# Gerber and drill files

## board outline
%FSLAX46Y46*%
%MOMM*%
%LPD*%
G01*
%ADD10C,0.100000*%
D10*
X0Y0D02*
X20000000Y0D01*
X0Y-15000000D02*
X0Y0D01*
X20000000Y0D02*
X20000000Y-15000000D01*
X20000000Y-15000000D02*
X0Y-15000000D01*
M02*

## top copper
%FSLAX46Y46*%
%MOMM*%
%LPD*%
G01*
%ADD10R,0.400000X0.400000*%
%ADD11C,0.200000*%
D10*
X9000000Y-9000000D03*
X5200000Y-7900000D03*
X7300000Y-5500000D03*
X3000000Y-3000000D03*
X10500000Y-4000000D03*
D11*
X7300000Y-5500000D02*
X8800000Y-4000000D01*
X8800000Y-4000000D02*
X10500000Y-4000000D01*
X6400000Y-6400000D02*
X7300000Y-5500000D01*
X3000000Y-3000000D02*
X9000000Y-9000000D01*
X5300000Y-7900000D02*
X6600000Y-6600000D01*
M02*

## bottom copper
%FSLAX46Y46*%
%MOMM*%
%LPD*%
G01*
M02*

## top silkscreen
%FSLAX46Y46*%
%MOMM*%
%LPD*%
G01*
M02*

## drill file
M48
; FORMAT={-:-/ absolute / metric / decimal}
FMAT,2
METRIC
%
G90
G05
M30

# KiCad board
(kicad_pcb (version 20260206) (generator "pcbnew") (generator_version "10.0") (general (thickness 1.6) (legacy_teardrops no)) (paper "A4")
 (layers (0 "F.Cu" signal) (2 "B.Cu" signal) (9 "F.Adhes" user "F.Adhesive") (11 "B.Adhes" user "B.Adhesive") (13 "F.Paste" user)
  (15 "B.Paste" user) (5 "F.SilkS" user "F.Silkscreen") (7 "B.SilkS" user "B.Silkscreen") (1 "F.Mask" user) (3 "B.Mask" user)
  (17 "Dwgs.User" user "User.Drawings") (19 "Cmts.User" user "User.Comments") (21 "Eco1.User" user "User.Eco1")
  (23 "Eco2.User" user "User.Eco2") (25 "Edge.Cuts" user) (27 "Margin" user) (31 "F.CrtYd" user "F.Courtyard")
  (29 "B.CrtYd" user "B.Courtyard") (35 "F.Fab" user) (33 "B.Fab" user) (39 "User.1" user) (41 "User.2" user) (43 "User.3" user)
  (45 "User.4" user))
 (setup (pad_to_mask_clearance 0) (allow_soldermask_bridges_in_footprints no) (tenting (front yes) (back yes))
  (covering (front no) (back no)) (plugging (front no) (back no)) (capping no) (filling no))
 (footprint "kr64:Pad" (layer "F.Cu") (at 9 9)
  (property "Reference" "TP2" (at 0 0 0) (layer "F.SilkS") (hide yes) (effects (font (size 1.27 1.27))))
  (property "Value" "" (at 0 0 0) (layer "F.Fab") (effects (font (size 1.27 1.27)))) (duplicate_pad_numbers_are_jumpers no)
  (pad "1" smd rect (at 0 0) (size 0.4 0.4) (layers "F.Cu" "F.Mask" "F.Paste") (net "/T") (thermal_bridge_angle 45)))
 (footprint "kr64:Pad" (layer "F.Cu") (at 5.2 7.9)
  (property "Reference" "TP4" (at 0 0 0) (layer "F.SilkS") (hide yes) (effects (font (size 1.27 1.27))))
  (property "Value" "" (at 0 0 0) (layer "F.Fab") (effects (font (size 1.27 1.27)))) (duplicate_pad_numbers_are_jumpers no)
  (pad "1" smd rect (at 0 0) (size 0.4 0.4) (layers "F.Cu" "F.Mask" "F.Paste") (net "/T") (thermal_bridge_angle 45)))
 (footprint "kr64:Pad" (layer "F.Cu") (at 7.3 5.5)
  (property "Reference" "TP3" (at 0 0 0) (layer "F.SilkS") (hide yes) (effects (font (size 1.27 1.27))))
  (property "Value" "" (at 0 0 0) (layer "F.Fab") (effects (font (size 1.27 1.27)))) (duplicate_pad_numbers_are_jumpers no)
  (pad "1" smd rect (at 0 0) (size 0.4 0.4) (layers "F.Cu" "F.Mask" "F.Paste") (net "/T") (thermal_bridge_angle 45)))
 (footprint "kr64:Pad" (layer "F.Cu") (at 3 3)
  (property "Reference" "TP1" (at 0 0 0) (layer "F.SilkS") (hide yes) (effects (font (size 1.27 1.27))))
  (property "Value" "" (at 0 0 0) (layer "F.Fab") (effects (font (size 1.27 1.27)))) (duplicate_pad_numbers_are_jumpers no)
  (pad "1" smd rect (at 0 0) (size 0.4 0.4) (layers "F.Cu" "F.Mask" "F.Paste") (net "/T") (thermal_bridge_angle 45)))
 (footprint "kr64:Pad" (layer "F.Cu") (at 10.5 4)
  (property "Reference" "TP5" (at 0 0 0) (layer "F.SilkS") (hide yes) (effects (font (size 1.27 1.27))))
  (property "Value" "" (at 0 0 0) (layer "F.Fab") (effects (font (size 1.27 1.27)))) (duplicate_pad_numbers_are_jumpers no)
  (pad "1" smd rect (at 0 0) (size 0.4 0.4) (layers "F.Cu" "F.Mask" "F.Paste") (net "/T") (thermal_bridge_angle 45)))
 (gr_line (start 0 0) (end 20 0) (stroke (width 0.1) (type default)) (layer "Edge.Cuts"))
 (gr_line (start 0 15) (end 0 0) (stroke (width 0.1) (type default)) (layer "Edge.Cuts"))
 (gr_line (start 20 0) (end 20 15) (stroke (width 0.1) (type default)) (layer "Edge.Cuts"))
 (gr_line (start 20 15) (end 0 15) (stroke (width 0.1) (type default)) (layer "Edge.Cuts"))
 (segment (start 7.3 5.5) (end 8.8 4) (width 0.2) (layer "F.Cu") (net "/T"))
 (segment (start 8.8 4) (end 10.5 4) (width 0.2) (layer "F.Cu") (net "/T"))
 (segment (start 6.4 6.4) (end 7.3 5.5) (width 0.2) (layer "F.Cu") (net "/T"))
 (segment (start 3 3) (end 9 9) (width 0.2) (layer "F.Cu") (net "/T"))
 (segment (start 5.3 7.9) (end 6.6 6.6) (width 0.2) (layer "F.Cu") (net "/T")))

